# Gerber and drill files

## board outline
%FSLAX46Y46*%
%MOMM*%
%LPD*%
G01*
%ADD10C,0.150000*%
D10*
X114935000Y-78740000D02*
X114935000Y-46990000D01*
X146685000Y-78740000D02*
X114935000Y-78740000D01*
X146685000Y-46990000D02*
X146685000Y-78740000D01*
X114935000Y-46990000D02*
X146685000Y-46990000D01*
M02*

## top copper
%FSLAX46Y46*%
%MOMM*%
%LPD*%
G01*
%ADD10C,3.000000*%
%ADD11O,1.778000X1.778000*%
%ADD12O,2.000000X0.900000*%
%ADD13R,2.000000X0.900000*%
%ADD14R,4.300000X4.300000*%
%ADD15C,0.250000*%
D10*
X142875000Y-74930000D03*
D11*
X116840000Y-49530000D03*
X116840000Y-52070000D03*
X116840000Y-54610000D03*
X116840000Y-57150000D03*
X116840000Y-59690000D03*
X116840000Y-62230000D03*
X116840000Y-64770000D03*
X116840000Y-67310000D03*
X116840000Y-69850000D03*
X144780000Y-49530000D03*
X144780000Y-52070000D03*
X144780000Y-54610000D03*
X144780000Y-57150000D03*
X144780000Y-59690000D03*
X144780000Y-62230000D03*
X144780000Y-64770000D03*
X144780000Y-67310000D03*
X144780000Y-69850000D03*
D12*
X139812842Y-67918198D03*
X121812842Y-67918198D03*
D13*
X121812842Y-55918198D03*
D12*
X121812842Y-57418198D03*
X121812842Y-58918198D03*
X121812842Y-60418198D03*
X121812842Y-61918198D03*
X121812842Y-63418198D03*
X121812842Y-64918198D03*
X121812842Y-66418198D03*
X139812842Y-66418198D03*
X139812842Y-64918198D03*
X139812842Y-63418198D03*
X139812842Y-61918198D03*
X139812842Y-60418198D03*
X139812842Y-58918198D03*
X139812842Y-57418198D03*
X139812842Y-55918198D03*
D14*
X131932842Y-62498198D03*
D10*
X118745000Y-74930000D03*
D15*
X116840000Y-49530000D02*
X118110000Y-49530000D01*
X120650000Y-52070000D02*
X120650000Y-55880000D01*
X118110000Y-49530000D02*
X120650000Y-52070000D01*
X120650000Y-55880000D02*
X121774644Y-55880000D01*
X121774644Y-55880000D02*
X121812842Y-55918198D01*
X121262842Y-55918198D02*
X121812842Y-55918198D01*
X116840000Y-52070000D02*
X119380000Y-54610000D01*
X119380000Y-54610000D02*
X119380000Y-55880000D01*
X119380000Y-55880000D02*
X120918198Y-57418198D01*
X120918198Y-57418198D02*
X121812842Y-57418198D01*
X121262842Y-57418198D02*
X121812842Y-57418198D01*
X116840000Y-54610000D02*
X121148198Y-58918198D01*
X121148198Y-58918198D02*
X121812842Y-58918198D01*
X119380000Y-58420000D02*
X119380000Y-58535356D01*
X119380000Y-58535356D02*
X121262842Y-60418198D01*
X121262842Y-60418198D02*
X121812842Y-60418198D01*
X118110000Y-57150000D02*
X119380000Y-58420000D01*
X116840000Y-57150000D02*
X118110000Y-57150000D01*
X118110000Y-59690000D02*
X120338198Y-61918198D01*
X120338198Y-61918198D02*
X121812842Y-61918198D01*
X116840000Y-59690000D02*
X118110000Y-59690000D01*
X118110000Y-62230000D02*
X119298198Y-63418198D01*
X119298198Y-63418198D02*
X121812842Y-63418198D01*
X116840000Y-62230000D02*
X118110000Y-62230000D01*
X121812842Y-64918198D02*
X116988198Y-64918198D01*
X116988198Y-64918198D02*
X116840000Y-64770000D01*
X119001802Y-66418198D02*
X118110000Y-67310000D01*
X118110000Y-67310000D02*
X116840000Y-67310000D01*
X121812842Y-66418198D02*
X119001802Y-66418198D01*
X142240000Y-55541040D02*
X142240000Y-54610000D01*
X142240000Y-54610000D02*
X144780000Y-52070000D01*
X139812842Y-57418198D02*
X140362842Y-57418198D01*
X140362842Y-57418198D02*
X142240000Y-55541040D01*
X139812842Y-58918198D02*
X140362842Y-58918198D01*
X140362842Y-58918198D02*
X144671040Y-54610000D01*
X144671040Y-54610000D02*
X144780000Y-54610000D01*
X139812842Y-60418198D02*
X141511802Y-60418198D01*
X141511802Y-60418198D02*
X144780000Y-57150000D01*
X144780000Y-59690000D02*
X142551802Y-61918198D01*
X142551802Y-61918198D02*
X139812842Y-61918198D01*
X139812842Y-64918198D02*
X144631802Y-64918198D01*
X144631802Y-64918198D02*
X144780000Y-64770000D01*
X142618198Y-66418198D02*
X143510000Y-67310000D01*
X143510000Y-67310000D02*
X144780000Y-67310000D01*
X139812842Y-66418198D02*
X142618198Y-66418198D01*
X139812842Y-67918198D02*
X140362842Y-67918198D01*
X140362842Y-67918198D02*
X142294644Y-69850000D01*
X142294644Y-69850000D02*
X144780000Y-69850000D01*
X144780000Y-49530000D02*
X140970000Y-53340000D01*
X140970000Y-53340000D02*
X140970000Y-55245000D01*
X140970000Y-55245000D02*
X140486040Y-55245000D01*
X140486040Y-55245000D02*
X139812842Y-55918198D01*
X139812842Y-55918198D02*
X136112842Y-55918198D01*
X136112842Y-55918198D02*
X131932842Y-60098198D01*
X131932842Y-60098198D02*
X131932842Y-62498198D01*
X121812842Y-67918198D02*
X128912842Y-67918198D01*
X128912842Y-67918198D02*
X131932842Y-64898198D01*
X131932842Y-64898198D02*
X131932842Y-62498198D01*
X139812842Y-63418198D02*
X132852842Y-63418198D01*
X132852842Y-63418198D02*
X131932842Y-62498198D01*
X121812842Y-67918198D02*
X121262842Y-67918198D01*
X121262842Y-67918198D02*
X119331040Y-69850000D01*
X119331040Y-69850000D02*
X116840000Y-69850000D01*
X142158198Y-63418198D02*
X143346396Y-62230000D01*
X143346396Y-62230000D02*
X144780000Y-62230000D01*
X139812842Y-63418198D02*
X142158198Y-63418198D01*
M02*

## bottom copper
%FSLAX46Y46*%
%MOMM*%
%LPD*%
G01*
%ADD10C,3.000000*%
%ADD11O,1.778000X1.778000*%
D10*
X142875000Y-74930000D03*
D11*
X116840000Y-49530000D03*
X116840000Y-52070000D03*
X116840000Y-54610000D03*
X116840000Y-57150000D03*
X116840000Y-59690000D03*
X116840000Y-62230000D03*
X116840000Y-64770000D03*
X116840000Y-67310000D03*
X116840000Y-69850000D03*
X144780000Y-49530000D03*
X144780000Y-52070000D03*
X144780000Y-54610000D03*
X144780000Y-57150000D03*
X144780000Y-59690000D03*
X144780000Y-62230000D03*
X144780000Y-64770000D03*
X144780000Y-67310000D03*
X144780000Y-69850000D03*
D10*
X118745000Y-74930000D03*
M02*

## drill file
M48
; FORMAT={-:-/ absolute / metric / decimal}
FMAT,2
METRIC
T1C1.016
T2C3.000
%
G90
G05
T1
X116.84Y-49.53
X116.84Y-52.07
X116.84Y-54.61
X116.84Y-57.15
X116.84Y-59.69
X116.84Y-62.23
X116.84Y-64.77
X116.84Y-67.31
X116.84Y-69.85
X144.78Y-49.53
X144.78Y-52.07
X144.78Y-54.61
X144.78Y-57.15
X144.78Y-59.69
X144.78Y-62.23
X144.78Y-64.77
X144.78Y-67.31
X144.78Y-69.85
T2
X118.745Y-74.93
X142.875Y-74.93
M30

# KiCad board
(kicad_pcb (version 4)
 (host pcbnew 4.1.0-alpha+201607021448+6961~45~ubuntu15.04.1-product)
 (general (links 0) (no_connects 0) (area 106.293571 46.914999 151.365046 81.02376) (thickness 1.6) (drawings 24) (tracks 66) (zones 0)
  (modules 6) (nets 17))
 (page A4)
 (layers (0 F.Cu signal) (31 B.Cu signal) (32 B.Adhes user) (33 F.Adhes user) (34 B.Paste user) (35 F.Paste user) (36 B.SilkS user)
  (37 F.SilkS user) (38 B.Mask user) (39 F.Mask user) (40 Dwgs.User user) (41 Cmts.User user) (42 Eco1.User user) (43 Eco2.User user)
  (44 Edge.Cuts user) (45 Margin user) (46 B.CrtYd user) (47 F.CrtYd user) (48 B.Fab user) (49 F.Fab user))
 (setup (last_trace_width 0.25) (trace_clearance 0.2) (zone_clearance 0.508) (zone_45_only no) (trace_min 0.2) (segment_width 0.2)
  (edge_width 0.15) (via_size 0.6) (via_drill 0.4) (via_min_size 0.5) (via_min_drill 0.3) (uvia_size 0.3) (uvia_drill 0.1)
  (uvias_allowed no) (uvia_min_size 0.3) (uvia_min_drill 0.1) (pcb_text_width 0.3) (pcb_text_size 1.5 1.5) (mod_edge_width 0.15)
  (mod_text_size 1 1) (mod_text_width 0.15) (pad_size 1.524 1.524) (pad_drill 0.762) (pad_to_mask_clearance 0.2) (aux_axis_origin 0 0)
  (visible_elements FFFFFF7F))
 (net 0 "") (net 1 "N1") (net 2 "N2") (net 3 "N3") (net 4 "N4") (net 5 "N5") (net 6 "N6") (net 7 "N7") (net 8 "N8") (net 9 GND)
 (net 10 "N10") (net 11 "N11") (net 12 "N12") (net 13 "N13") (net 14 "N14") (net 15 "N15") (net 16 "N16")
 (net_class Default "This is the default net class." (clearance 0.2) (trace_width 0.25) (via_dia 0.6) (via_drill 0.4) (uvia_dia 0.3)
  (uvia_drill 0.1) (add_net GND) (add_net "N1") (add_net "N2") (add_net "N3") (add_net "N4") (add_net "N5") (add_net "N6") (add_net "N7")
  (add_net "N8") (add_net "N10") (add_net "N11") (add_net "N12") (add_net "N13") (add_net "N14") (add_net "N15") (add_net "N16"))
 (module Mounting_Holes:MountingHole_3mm (layer F.Cu) (at 142.875 74.93)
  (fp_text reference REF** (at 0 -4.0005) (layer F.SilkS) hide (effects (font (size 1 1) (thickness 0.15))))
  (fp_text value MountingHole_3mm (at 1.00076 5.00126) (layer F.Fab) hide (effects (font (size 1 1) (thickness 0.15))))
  (pad 1 thru_hole circle (at 0 0) (size 3 3) (drill 3) (layers)))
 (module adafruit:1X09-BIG (layer F.Cu) (at 116.84 59.69 270)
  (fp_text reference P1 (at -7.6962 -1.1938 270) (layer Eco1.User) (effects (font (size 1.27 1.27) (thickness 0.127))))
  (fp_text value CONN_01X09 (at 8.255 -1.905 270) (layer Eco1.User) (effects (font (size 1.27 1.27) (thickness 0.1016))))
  (pad 1 thru_hole oval (at -10.16 0) (size 1.778 1.778) (drill 1.016) (layers *.Cu *.Mask) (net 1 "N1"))
  (pad 2 thru_hole oval (at -7.62 0) (size 1.778 1.778) (drill 1.016) (layers *.Cu *.Mask) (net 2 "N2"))
  (pad 3 thru_hole oval (at -5.08 0) (size 1.778 1.778) (drill 1.016) (layers *.Cu *.Mask) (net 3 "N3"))
  (pad 4 thru_hole oval (at -2.54 0) (size 1.778 1.778) (drill 1.016) (layers *.Cu *.Mask) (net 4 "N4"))
  (pad 5 thru_hole oval (at 0 0) (size 1.778 1.778) (drill 1.016) (layers *.Cu *.Mask) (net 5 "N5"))
  (pad 6 thru_hole oval (at 2.54 0) (size 1.778 1.778) (drill 1.016) (layers *.Cu *.Mask) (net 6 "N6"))
  (pad 7 thru_hole oval (at 5.08 0) (size 1.778 1.778) (drill 1.016) (layers *.Cu *.Mask) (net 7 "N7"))
  (pad 8 thru_hole oval (at 7.62 0) (size 1.778 1.778) (drill 1.016) (layers *.Cu *.Mask) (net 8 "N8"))
  (pad 9 thru_hole oval (at 10.16 0) (size 1.778 1.778) (drill 1.016) (layers *.Cu *.Mask) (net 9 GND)))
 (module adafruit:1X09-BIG (layer F.Cu) (at 144.78 59.69 270)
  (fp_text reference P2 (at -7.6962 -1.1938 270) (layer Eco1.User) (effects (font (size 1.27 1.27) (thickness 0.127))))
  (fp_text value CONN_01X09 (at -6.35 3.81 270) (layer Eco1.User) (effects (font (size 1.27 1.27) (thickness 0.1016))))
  (pad 1 thru_hole oval (at -10.16 0) (size 1.778 1.778) (drill 1.016) (layers *.Cu *.Mask) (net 9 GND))
  (pad 2 thru_hole oval (at -7.62 0) (size 1.778 1.778) (drill 1.016) (layers *.Cu *.Mask) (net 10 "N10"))
  (pad 3 thru_hole oval (at -5.08 0) (size 1.778 1.778) (drill 1.016) (layers *.Cu *.Mask) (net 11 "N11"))
  (pad 4 thru_hole oval (at -2.54 0) (size 1.778 1.778) (drill 1.016) (layers *.Cu *.Mask) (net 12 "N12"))
  (pad 5 thru_hole oval (at 0 0) (size 1.778 1.778) (drill 1.016) (layers *.Cu *.Mask) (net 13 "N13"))
  (pad 6 thru_hole oval (at 2.54 0) (size 1.778 1.778) (drill 1.016) (layers *.Cu *.Mask) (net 9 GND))
  (pad 7 thru_hole oval (at 5.08 0) (size 1.778 1.778) (drill 1.016) (layers *.Cu *.Mask) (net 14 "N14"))
  (pad 8 thru_hole oval (at 7.62 0) (size 1.778 1.778) (drill 1.016) (layers *.Cu *.Mask) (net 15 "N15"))
  (pad 9 thru_hole oval (at 10.16 0) (size 1.778 1.778) (drill 1.016) (layers *.Cu *.Mask) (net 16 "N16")))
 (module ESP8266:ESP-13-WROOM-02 (layer F.Cu) (at 121.812842 55.918198)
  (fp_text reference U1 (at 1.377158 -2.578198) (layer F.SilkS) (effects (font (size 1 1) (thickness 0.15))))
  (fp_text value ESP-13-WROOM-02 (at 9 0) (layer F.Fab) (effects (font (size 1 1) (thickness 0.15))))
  (pad 10 smd oval (at 18 12) (size 2 0.9) (layers F.Cu F.Paste F.Mask) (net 16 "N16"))
  (pad 9 smd oval (at 0 12) (size 2 0.9) (layers F.Cu F.Paste F.Mask) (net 9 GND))
  (pad 1 smd rect (at 0 0) (size 2 0.9) (layers F.Cu F.Paste F.Mask) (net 1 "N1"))
  (pad 2 smd oval (at 0 1.5) (size 2 0.9) (layers F.Cu F.Paste F.Mask) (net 2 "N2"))
  (pad 3 smd oval (at 0 3) (size 2 0.9) (layers F.Cu F.Paste F.Mask) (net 3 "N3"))
  (pad 4 smd oval (at 0 4.5) (size 2 0.9) (layers F.Cu F.Paste F.Mask) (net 4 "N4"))
  (pad 5 smd oval (at 0 6) (size 2 0.9) (layers F.Cu F.Paste F.Mask) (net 5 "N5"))
  (pad 6 smd oval (at 0 7.5) (size 2 0.9) (layers F.Cu F.Paste F.Mask) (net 6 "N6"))
  (pad 7 smd oval (at 0 9) (size 2 0.9) (layers F.Cu F.Paste F.Mask) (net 7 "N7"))
  (pad 8 smd oval (at 0 10.5) (size 2 0.9) (layers F.Cu F.Paste F.Mask) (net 8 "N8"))
  (pad 11 smd oval (at 18 10.5) (size 2 0.9) (layers F.Cu F.Paste F.Mask) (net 15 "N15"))
  (pad 12 smd oval (at 18 9) (size 2 0.9) (layers F.Cu F.Paste F.Mask) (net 14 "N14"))
  (pad 13 smd oval (at 18 7.5) (size 2 0.9) (layers F.Cu F.Paste F.Mask) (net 9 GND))
  (pad 14 smd oval (at 18 6) (size 2 0.9) (layers F.Cu F.Paste F.Mask) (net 13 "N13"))
  (pad 15 smd oval (at 18 4.5) (size 2 0.9) (layers F.Cu F.Paste F.Mask) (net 12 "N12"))
  (pad 16 smd oval (at 18 3) (size 2 0.9) (layers F.Cu F.Paste F.Mask) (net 11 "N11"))
  (pad 17 smd oval (at 18 1.5) (size 2 0.9) (layers F.Cu F.Paste F.Mask) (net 10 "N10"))
  (pad 18 smd oval (at 18 0) (size 2 0.9) (layers F.Cu F.Paste F.Mask) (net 9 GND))
  (pad PAD smd rect (at 10.12 6.58) (size 4.3 4.3) (layers F.Cu F.Paste F.Mask) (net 9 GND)))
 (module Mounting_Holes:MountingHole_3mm (layer F.Cu) (at 118.745 74.93)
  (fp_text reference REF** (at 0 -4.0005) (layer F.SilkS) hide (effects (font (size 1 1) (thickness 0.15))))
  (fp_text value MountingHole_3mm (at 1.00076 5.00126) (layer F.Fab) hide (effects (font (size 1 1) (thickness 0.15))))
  (pad 1 thru_hole circle (at 0 0) (size 3 3) (drill 3) (layers)))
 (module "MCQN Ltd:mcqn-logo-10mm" (layer F.Cu) (at 134.62 76.2)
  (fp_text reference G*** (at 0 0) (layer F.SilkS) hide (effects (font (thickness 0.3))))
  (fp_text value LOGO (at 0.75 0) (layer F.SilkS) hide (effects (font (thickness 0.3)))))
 (gr_line (start 114.935 78.74) (end 114.935 46.99) (layer Edge.Cuts) (width 0.15))
 (gr_line (start 146.685 78.74) (end 114.935 78.74) (layer Edge.Cuts) (width 0.15))
 (gr_line (start 146.685 46.99) (end 146.685 78.74) (layer Edge.Cuts) (width 0.15))
 (gr_line (start 114.935 46.99) (end 146.685 46.99) (layer Edge.Cuts) (width 0.15))
 (segment (start 116.84 49.53) (end 118.11 49.53) (width 0.25) (layer F.Cu) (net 1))
 (segment (start 120.65 52.07) (end 120.65 55.88) (width 0.25) (layer F.Cu) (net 1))
 (segment (start 118.11 49.53) (end 120.65 52.07) (width 0.25) (layer F.Cu) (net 1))
 (segment (start 120.65 55.88) (end 121.774644 55.88) (width 0.25) (layer F.Cu) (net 1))
 (segment (start 121.774644 55.88) (end 121.812842 55.918198) (width 0.25) (layer F.Cu) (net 1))
 (segment (start 121.262842 55.918198) (end 121.812842 55.918198) (width 0.25) (layer F.Cu) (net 1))
 (segment (start 116.84 52.07) (end 119.38 54.61) (width 0.25) (layer F.Cu) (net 2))
 (segment (start 119.38 54.61) (end 119.38 55.88) (width 0.25) (layer F.Cu) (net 2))
 (segment (start 119.38 55.88) (end 120.918198 57.418198) (width 0.25) (layer F.Cu) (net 2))
 (segment (start 120.918198 57.418198) (end 121.812842 57.418198) (width 0.25) (layer F.Cu) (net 2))
 (segment (start 121.262842 57.418198) (end 121.812842 57.418198) (width 0.25) (layer F.Cu) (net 2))
 (segment (start 116.84 54.61) (end 121.148198 58.918198) (width 0.25) (layer F.Cu) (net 3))
 (segment (start 121.148198 58.918198) (end 121.812842 58.918198) (width 0.25) (layer F.Cu) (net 3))
 (segment (start 119.38 58.42) (end 119.38 58.535356) (width 0.25) (layer F.Cu) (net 4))
 (segment (start 119.38 58.535356) (end 121.262842 60.418198) (width 0.25) (layer F.Cu) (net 4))
 (segment (start 121.262842 60.418198) (end 121.812842 60.418198) (width 0.25) (layer F.Cu) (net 4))
 (segment (start 118.11 57.15) (end 119.38 58.42) (width 0.25) (layer F.Cu) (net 4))
 (segment (start 116.84 57.15) (end 118.11 57.15) (width 0.25) (layer F.Cu) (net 4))
 (segment (start 118.11 59.69) (end 120.338198 61.918198) (width 0.25) (layer F.Cu) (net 5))
 (segment (start 120.338198 61.918198) (end 121.812842 61.918198) (width 0.25) (layer F.Cu) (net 5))
 (segment (start 116.84 59.69) (end 118.11 59.69) (width 0.25) (layer F.Cu) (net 5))
 (segment (start 118.11 62.23) (end 119.298198 63.418198) (width 0.25) (layer F.Cu) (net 6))
 (segment (start 119.298198 63.418198) (end 121.812842 63.418198) (width 0.25) (layer F.Cu) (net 6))
 (segment (start 116.84 62.23) (end 118.11 62.23) (width 0.25) (layer F.Cu) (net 6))
 (segment (start 121.812842 64.918198) (end 116.988198 64.918198) (width 0.25) (layer F.Cu) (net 7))
 (segment (start 116.988198 64.918198) (end 116.84 64.77) (width 0.25) (layer F.Cu) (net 7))
 (segment (start 119.001802 66.418198) (end 118.11 67.31) (width 0.25) (layer F.Cu) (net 8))
 (segment (start 118.11 67.31) (end 116.84 67.31) (width 0.25) (layer F.Cu) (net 8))
 (segment (start 121.812842 66.418198) (end 119.001802 66.418198) (width 0.25) (layer F.Cu) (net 8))
 (segment (start 142.24 55.54104) (end 142.24 54.61) (width 0.25) (layer F.Cu) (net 10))
 (segment (start 142.24 54.61) (end 144.78 52.07) (width 0.25) (layer F.Cu) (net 10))
 (segment (start 139.812842 57.418198) (end 140.362842 57.418198) (width 0.25) (layer F.Cu) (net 10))
 (segment (start 140.362842 57.418198) (end 142.24 55.54104) (width 0.25) (layer F.Cu) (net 10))
 (segment (start 139.812842 58.918198) (end 140.362842 58.918198) (width 0.25) (layer F.Cu) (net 11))
 (segment (start 140.362842 58.918198) (end 144.67104 54.61) (width 0.25) (layer F.Cu) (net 11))
 (segment (start 144.67104 54.61) (end 144.78 54.61) (width 0.25) (layer F.Cu) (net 11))
 (segment (start 139.812842 60.418198) (end 141.511802 60.418198) (width 0.25) (layer F.Cu) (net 12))
 (segment (start 141.511802 60.418198) (end 144.78 57.15) (width 0.25) (layer F.Cu) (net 12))
 (segment (start 144.78 59.69) (end 142.551802 61.918198) (width 0.25) (layer F.Cu) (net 13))
 (segment (start 142.551802 61.918198) (end 139.812842 61.918198) (width 0.25) (layer F.Cu) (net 13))
 (segment (start 139.812842 64.918198) (end 144.631802 64.918198) (width 0.25) (layer F.Cu) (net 14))
 (segment (start 144.631802 64.918198) (end 144.78 64.77) (width 0.25) (layer F.Cu) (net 14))
 (segment (start 142.618198 66.418198) (end 143.51 67.31) (width 0.25) (layer F.Cu) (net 15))
 (segment (start 143.51 67.31) (end 144.78 67.31) (width 0.25) (layer F.Cu) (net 15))
 (segment (start 139.812842 66.418198) (end 142.618198 66.418198) (width 0.25) (layer F.Cu) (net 15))
 (segment (start 139.812842 67.918198) (end 140.362842 67.918198) (width 0.25) (layer F.Cu) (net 16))
 (segment (start 140.362842 67.918198) (end 142.294644 69.85) (width 0.25) (layer F.Cu) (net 16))
 (segment (start 142.294644 69.85) (end 144.78 69.85) (width 0.25) (layer F.Cu) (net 16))
 (segment (start 144.78 49.53) (end 140.97 53.34) (width 0.25) (layer F.Cu) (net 9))
 (segment (start 140.97 53.34) (end 140.97 55.245) (width 0.25) (layer F.Cu) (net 9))
 (segment (start 140.97 55.245) (end 140.48604 55.245) (width 0.25) (layer F.Cu) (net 9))
 (segment (start 140.48604 55.245) (end 139.812842 55.918198) (width 0.25) (layer F.Cu) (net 9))
 (segment (start 139.812842 55.918198) (end 136.112842 55.918198) (width 0.25) (layer F.Cu) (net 9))
 (segment (start 136.112842 55.918198) (end 131.932842 60.098198) (width 0.25) (layer F.Cu) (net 9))
 (segment (start 131.932842 60.098198) (end 131.932842 62.498198) (width 0.25) (layer F.Cu) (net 9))
 (segment (start 121.812842 67.918198) (end 128.912842 67.918198) (width 0.25) (layer F.Cu) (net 9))
 (segment (start 128.912842 67.918198) (end 131.932842 64.898198) (width 0.25) (layer F.Cu) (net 9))
 (segment (start 131.932842 64.898198) (end 131.932842 62.498198) (width 0.25) (layer F.Cu) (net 9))
 (segment (start 139.812842 63.418198) (end 132.852842 63.418198) (width 0.25) (layer F.Cu) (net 9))
 (segment (start 132.852842 63.418198) (end 131.932842 62.498198) (width 0.25) (layer F.Cu) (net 9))
 (segment (start 121.812842 67.918198) (end 121.262842 67.918198) (width 0.25) (layer F.Cu) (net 9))
 (segment (start 121.262842 67.918198) (end 119.33104 69.85) (width 0.25) (layer F.Cu) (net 9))
 (segment (start 119.33104 69.85) (end 116.84 69.85) (width 0.25) (layer F.Cu) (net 9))
 (segment (start 142.158198 63.418198) (end 143.346396 62.23) (width 0.25) (layer F.Cu) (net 9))
 (segment (start 143.346396 62.23) (end 144.78 62.23) (width 0.25) (layer F.Cu) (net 9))
 (segment (start 139.812842 63.418198) (end 142.158198 63.418198) (width 0.25) (layer F.Cu) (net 9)))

